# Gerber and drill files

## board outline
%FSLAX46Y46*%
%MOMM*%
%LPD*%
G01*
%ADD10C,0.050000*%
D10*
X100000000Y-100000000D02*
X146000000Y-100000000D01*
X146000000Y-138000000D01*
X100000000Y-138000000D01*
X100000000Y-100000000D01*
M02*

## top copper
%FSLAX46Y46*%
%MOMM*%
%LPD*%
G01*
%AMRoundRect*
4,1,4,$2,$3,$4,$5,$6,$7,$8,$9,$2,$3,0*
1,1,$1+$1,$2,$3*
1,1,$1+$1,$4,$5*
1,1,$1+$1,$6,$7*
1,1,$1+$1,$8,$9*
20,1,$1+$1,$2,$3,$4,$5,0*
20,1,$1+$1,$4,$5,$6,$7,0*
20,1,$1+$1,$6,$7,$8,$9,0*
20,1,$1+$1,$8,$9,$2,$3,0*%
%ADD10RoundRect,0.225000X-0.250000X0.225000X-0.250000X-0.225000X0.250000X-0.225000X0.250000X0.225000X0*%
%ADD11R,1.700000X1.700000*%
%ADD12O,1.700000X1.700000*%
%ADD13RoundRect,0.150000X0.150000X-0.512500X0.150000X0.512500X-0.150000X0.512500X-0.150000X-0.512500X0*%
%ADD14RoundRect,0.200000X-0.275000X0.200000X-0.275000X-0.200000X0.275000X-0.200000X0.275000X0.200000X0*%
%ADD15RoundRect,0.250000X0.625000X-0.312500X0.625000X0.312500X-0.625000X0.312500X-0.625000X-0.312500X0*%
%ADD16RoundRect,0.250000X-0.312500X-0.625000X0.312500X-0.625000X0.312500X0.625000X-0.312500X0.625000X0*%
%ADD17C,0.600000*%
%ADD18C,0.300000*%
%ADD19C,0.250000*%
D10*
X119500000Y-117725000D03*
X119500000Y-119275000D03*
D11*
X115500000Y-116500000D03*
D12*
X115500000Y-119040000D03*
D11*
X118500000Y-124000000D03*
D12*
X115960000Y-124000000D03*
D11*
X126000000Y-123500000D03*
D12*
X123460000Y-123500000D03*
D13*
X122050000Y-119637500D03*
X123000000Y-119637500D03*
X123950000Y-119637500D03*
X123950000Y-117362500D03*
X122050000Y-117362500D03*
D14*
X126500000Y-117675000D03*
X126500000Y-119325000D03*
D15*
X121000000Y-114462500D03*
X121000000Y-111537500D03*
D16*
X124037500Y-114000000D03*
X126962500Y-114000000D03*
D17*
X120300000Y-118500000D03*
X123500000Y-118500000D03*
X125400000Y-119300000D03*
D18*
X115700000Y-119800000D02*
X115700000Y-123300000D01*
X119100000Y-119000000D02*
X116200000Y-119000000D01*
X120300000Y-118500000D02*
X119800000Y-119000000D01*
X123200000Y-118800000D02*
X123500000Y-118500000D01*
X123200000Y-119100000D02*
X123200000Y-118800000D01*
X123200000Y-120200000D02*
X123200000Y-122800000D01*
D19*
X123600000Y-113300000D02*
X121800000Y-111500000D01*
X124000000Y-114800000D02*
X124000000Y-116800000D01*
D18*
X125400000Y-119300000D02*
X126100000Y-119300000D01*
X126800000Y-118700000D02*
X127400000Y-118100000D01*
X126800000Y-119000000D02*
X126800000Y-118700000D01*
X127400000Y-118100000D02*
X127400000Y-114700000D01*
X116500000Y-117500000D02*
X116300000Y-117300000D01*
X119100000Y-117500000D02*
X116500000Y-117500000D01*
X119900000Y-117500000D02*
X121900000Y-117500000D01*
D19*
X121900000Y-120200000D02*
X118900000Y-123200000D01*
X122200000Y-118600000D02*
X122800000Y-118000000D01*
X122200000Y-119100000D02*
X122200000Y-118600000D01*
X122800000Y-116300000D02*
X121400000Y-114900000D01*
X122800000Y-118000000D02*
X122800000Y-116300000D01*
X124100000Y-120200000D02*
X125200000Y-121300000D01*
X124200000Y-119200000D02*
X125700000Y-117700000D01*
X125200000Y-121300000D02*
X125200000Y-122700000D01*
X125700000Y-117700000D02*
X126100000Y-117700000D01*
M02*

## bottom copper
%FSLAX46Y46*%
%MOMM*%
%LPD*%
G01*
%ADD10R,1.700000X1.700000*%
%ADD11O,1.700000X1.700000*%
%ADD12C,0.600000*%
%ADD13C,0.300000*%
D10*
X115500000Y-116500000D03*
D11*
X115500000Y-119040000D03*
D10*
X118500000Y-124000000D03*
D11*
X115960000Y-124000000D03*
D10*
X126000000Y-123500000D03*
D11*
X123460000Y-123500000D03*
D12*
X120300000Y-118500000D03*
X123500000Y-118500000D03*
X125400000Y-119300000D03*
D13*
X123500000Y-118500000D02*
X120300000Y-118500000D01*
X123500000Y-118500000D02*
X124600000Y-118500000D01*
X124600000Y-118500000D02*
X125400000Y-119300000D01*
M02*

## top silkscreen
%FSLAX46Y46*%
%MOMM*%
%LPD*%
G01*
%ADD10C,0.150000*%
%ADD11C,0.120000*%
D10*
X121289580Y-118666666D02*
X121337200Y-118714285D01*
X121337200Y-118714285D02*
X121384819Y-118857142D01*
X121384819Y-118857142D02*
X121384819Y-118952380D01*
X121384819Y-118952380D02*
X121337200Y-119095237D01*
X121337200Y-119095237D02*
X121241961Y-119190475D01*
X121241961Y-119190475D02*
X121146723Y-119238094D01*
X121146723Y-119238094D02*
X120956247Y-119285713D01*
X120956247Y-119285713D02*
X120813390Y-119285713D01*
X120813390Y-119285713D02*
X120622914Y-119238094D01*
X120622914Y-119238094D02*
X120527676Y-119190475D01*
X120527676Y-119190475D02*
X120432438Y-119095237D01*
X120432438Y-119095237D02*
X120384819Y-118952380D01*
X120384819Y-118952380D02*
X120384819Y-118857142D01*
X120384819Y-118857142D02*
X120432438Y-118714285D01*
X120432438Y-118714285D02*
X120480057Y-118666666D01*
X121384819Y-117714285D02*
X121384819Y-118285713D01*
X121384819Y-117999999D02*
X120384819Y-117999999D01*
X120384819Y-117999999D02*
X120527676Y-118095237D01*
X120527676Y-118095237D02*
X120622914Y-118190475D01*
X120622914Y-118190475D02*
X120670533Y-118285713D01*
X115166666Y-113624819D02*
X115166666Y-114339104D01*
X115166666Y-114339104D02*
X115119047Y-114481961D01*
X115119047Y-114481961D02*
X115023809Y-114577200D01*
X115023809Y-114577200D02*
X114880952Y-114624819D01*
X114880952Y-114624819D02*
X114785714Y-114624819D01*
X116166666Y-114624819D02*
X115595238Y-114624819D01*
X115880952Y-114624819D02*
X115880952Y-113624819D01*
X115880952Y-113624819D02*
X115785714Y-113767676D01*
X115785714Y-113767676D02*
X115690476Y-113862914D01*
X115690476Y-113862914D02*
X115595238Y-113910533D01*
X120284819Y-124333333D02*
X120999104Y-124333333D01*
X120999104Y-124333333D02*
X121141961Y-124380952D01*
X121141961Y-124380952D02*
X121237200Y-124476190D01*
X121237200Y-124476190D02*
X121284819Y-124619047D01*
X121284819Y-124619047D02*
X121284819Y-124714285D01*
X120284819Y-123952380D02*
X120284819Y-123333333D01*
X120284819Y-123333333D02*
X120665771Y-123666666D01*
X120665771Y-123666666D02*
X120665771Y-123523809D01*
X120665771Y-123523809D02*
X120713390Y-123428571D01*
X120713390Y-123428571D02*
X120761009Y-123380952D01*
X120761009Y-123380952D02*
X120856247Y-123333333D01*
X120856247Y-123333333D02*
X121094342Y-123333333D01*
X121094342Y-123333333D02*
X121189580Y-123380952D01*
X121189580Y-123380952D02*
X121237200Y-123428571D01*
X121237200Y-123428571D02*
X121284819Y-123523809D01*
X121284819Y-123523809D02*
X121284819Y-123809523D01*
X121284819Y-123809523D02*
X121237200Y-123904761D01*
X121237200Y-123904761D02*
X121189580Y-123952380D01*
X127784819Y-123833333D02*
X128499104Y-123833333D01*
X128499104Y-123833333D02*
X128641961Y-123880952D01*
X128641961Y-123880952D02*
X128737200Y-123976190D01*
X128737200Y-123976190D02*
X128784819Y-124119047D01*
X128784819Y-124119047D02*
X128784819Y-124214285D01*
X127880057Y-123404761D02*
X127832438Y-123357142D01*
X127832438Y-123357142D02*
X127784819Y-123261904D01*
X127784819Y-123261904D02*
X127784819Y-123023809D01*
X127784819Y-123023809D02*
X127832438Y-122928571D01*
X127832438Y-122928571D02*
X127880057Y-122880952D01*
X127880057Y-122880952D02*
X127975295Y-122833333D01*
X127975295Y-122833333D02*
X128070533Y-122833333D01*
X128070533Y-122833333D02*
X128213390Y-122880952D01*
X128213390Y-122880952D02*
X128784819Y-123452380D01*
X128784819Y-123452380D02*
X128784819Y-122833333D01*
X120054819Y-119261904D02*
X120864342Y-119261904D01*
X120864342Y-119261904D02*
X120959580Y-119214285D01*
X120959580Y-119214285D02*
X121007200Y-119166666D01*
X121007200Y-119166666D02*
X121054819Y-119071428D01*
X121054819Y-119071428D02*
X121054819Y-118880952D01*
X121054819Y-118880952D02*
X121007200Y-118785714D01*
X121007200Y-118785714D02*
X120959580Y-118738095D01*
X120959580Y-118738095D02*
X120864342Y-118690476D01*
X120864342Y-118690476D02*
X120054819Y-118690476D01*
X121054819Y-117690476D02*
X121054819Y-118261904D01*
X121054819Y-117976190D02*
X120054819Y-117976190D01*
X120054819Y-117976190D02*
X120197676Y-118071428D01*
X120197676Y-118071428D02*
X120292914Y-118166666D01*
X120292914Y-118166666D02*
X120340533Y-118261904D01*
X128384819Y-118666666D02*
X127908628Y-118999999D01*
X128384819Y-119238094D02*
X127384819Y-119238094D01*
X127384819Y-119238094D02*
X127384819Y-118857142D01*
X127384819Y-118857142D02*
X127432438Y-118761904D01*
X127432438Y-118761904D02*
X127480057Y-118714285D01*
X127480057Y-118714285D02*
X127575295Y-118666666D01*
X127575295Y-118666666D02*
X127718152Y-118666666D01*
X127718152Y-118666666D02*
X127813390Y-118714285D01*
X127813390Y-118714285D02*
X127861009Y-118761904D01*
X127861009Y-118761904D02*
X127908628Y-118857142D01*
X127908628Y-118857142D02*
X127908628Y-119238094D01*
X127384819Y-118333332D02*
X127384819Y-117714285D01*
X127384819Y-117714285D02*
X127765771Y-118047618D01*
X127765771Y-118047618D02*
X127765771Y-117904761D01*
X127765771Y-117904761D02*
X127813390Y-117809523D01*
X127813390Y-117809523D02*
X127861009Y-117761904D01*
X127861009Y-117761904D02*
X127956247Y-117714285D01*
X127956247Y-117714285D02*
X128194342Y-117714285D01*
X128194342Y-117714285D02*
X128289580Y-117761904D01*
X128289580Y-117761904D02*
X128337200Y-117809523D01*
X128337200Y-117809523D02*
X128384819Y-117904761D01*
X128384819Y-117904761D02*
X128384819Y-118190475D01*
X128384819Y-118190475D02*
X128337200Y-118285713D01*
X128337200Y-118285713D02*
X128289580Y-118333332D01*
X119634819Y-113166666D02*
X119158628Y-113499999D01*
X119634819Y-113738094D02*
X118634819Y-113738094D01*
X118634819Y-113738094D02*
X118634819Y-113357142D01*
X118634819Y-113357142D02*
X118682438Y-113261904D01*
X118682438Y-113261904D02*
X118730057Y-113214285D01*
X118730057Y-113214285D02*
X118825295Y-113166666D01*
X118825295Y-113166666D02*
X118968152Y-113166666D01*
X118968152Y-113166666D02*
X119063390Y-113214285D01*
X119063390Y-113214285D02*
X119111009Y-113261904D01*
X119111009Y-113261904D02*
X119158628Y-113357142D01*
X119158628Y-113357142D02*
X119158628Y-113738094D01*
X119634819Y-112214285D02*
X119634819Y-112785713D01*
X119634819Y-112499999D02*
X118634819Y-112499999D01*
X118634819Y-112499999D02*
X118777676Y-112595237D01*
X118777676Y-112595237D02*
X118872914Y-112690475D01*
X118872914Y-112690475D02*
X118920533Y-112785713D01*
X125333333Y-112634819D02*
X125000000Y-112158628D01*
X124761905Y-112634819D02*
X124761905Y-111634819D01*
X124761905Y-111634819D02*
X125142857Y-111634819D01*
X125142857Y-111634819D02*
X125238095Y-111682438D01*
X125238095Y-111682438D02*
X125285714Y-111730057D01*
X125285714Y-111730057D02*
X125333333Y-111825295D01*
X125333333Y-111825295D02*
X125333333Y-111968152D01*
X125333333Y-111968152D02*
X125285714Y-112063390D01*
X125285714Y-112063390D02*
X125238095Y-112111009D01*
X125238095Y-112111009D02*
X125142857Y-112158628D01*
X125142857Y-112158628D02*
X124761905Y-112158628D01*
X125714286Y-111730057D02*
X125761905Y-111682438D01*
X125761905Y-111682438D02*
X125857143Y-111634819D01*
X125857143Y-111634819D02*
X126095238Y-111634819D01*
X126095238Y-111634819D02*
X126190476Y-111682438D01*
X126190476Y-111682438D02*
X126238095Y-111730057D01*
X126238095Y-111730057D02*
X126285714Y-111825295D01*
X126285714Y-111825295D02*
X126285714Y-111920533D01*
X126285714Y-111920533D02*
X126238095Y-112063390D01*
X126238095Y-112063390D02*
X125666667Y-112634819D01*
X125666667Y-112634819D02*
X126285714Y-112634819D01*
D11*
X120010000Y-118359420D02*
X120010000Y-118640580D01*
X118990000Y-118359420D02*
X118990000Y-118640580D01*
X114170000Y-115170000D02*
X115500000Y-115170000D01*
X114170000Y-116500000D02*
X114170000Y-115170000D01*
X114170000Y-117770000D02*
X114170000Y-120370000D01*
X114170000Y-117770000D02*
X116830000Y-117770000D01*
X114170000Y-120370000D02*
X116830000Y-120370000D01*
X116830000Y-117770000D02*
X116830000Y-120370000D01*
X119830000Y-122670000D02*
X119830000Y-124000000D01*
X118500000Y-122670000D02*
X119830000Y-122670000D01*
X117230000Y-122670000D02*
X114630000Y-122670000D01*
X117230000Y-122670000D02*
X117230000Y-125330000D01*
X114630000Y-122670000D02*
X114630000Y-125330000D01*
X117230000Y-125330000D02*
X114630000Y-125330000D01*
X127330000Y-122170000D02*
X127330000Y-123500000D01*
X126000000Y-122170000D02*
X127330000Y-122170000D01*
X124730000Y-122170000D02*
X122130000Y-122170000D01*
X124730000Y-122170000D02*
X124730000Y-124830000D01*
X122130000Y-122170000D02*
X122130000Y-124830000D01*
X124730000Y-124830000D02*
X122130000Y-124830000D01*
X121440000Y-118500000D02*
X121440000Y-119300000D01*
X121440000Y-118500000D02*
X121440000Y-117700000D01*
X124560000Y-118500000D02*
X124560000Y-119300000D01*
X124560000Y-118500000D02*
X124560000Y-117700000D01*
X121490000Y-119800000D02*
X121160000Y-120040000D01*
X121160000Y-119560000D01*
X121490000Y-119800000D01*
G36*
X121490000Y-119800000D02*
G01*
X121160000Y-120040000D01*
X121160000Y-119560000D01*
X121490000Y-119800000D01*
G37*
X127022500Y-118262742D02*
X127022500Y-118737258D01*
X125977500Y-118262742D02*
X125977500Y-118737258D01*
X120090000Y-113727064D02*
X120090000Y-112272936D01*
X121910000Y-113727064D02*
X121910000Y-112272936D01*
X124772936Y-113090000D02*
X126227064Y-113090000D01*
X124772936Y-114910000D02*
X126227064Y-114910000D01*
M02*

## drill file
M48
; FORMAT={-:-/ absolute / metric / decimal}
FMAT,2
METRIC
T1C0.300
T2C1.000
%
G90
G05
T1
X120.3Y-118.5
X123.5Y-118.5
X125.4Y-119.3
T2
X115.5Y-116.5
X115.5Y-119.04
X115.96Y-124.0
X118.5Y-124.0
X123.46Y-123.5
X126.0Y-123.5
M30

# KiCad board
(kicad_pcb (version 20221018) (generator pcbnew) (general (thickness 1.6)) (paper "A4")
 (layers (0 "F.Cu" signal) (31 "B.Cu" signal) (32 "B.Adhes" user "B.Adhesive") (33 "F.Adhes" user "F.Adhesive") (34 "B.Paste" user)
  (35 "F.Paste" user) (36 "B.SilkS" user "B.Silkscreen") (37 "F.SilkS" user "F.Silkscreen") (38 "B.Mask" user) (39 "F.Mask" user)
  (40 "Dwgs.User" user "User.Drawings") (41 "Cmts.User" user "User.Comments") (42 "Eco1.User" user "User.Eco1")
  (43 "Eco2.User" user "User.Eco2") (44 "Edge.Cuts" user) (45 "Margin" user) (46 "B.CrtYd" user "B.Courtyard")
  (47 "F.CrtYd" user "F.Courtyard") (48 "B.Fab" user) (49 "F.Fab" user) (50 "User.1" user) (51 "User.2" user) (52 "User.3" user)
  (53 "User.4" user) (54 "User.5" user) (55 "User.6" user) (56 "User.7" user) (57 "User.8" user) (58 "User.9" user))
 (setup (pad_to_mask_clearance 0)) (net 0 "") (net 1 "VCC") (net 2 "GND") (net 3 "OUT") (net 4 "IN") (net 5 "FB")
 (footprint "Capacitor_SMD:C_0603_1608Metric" (layer "F.Cu") (at 119.5 118.5 -90)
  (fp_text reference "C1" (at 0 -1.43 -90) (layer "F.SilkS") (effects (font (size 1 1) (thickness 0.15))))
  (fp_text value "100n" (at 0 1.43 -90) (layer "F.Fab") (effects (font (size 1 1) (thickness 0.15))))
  (fp_line (start -0.14058 -0.51) (end 0.14058 -0.51) (stroke (width 0.12) (type solid)) (layer "F.SilkS"))
  (fp_line (start -0.14058 0.51) (end 0.14058 0.51) (stroke (width 0.12) (type solid)) (layer "F.SilkS"))
  (pad "1" smd roundrect (at -0.775 0 270) (size 0.9 0.95) (layers "F.Cu" "F.Paste" "F.Mask") (roundrect_rratio 0.25) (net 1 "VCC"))
  (pad "2" smd roundrect (at 0.775 0 270) (size 0.9 0.95) (layers "F.Cu" "F.Paste" "F.Mask") (roundrect_rratio 0.25) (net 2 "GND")))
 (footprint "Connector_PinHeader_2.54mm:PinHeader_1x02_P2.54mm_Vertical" (layer "F.Cu") (at 115.5 116.5)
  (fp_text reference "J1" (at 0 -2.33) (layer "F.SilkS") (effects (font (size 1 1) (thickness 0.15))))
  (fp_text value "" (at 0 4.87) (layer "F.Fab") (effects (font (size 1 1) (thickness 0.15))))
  (fp_line (start -1.33 -1.33) (end 0 -1.33) (stroke (width 0.12) (type solid)) (layer "F.SilkS"))
  (fp_line (start -1.33 0) (end -1.33 -1.33) (stroke (width 0.12) (type solid)) (layer "F.SilkS"))
  (fp_line (start -1.33 1.27) (end -1.33 3.87) (stroke (width 0.12) (type solid)) (layer "F.SilkS"))
  (fp_line (start -1.33 1.27) (end 1.33 1.27) (stroke (width 0.12) (type solid)) (layer "F.SilkS"))
  (fp_line (start -1.33 3.87) (end 1.33 3.87) (stroke (width 0.12) (type solid)) (layer "F.SilkS"))
  (fp_line (start 1.33 1.27) (end 1.33 3.87) (stroke (width 0.12) (type solid)) (layer "F.SilkS"))
  (pad "1" thru_hole rect (at 0 0) (size 1.7 1.7) (drill 1) (layers "*.Cu" "*.Mask") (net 1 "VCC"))
  (pad "2" thru_hole oval (at 0 2.54) (size 1.7 1.7) (drill 1) (layers "*.Cu" "*.Mask") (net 2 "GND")))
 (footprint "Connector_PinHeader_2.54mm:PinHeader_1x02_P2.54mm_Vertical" (layer "F.Cu") (at 118.5 124 -90)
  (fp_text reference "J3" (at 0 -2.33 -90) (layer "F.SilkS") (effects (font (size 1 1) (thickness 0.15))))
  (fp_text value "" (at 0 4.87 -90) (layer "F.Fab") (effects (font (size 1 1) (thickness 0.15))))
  (fp_line (start -1.33 -1.33) (end 0 -1.33) (stroke (width 0.12) (type solid)) (layer "F.SilkS"))
  (fp_line (start -1.33 0) (end -1.33 -1.33) (stroke (width 0.12) (type solid)) (layer "F.SilkS"))
  (fp_line (start -1.33 1.27) (end -1.33 3.87) (stroke (width 0.12) (type solid)) (layer "F.SilkS"))
  (fp_line (start -1.33 1.27) (end 1.33 1.27) (stroke (width 0.12) (type solid)) (layer "F.SilkS"))
  (fp_line (start -1.33 3.87) (end 1.33 3.87) (stroke (width 0.12) (type solid)) (layer "F.SilkS"))
  (fp_line (start 1.33 1.27) (end 1.33 3.87) (stroke (width 0.12) (type solid)) (layer "F.SilkS"))
  (pad "1" thru_hole rect (at 0 0 270) (size 1.7 1.7) (drill 1) (layers "*.Cu" "*.Mask") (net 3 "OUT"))
  (pad "2" thru_hole oval (at 0 2.54 270) (size 1.7 1.7) (drill 1) (layers "*.Cu" "*.Mask") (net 2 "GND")))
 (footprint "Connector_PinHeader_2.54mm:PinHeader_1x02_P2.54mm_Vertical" (layer "F.Cu") (at 126 123.5 -90)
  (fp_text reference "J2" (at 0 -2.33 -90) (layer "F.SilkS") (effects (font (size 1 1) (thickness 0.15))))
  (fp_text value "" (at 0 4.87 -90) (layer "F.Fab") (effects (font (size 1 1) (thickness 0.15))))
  (fp_line (start -1.33 -1.33) (end 0 -1.33) (stroke (width 0.12) (type solid)) (layer "F.SilkS"))
  (fp_line (start -1.33 0) (end -1.33 -1.33) (stroke (width 0.12) (type solid)) (layer "F.SilkS"))
  (fp_line (start -1.33 1.27) (end -1.33 3.87) (stroke (width 0.12) (type solid)) (layer "F.SilkS"))
  (fp_line (start -1.33 1.27) (end 1.33 1.27) (stroke (width 0.12) (type solid)) (layer "F.SilkS"))
  (fp_line (start -1.33 3.87) (end 1.33 3.87) (stroke (width 0.12) (type solid)) (layer "F.SilkS"))
  (fp_line (start 1.33 1.27) (end 1.33 3.87) (stroke (width 0.12) (type solid)) (layer "F.SilkS"))
  (pad "1" thru_hole rect (at 0 0 270) (size 1.7 1.7) (drill 1) (layers "*.Cu" "*.Mask") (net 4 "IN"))
  (pad "2" thru_hole oval (at 0 2.54 270) (size 1.7 1.7) (drill 1) (layers "*.Cu" "*.Mask") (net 2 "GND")))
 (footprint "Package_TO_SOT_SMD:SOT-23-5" (layer "F.Cu") (at 123 118.5 90)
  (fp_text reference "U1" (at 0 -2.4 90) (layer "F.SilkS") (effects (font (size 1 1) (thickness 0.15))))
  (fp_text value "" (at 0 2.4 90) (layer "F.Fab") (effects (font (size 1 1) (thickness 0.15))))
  (fp_line (start 0 -1.56) (end -0.8 -1.56) (stroke (width 0.12) (type solid)) (layer "F.SilkS"))
  (fp_line (start 0 -1.56) (end 0.8 -1.56) (stroke (width 0.12) (type solid)) (layer "F.SilkS"))
  (fp_line (start 0 1.56) (end -0.8 1.56) (stroke (width 0.12) (type solid)) (layer "F.SilkS"))
  (fp_line (start 0 1.56) (end 0.8 1.56) (stroke (width 0.12) (type solid)) (layer "F.SilkS"))
  (fp_poly
   (pts (xy -1.3 -1.51) (xy -1.54 -1.84) (xy -1.06 -1.84) (xy -1.3 -1.51)) (stroke (width 0.12) (type solid)) (fill solid) (layer "F.SilkS"))
  (pad "1" smd roundrect (at -1.1375 -0.95 90) (size 1.325 0.6) (layers "F.Cu" "F.Paste" "F.Mask") (roundrect_rratio 0.25) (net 3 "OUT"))
  (pad "2" smd roundrect (at -1.1375 0 90) (size 1.325 0.6) (layers "F.Cu" "F.Paste" "F.Mask") (roundrect_rratio 0.25) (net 2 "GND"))
  (pad "3" smd roundrect (at -1.1375 0.95 90) (size 1.325 0.6) (layers "F.Cu" "F.Paste" "F.Mask") (roundrect_rratio 0.25) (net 4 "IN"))
  (pad "4" smd roundrect (at 1.1375 0.95 90) (size 1.325 0.6) (layers "F.Cu" "F.Paste" "F.Mask") (roundrect_rratio 0.25) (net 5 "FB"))
  (pad "5" smd roundrect (at 1.1375 -0.95 90) (size 1.325 0.6) (layers "F.Cu" "F.Paste" "F.Mask") (roundrect_rratio 0.25) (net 1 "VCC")))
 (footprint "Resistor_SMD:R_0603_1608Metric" (layer "F.Cu") (at 126.5 118.5 -90)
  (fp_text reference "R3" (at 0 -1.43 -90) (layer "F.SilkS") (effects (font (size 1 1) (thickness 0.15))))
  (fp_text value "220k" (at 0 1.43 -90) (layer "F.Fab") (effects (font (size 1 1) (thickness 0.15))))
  (fp_line (start -0.237258 -0.5225) (end 0.237258 -0.5225) (stroke (width 0.12) (type solid)) (layer "F.SilkS"))
  (fp_line (start -0.237258 0.5225) (end 0.237258 0.5225) (stroke (width 0.12) (type solid)) (layer "F.SilkS"))
  (pad "1" smd roundrect (at -0.825 0 270) (size 0.8 0.95) (layers "F.Cu" "F.Paste" "F.Mask") (roundrect_rratio 0.25) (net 4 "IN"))
  (pad "2" smd roundrect (at 0.825 0 270) (size 0.8 0.95) (layers "F.Cu" "F.Paste" "F.Mask") (roundrect_rratio 0.25) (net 2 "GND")))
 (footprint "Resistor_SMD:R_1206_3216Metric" (layer "F.Cu") (at 121 113 90)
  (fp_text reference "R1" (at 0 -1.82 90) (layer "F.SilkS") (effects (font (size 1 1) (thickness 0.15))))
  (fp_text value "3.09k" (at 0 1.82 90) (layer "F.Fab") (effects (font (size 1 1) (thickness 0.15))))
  (fp_line (start -0.727064 -0.91) (end 0.727064 -0.91) (stroke (width 0.12) (type solid)) (layer "F.SilkS"))
  (fp_line (start -0.727064 0.91) (end 0.727064 0.91) (stroke (width 0.12) (type solid)) (layer "F.SilkS"))
  (pad "1" smd roundrect (at -1.4625 0 90) (size 1.125 1.75) (layers "F.Cu" "F.Paste" "F.Mask") (roundrect_rratio 0.222222) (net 3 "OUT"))
  (pad "2" smd roundrect (at 1.4625 0 90) (size 1.125 1.75) (layers "F.Cu" "F.Paste" "F.Mask") (roundrect_rratio 0.222222) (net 5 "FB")))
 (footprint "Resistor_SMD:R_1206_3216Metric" (layer "F.Cu") (at 125.5 114)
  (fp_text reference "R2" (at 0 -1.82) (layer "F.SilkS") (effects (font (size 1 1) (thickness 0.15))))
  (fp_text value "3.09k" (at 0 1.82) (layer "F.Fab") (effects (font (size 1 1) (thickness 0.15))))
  (fp_line (start -0.727064 -0.91) (end 0.727064 -0.91) (stroke (width 0.12) (type solid)) (layer "F.SilkS"))
  (fp_line (start -0.727064 0.91) (end 0.727064 0.91) (stroke (width 0.12) (type solid)) (layer "F.SilkS"))
  (pad "1" smd roundrect (at -1.4625 0) (size 1.125 1.75) (layers "F.Cu" "F.Paste" "F.Mask") (roundrect_rratio 0.222222) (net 5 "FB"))
  (pad "2" smd roundrect (at 1.4625 0) (size 1.125 1.75) (layers "F.Cu" "F.Paste" "F.Mask") (roundrect_rratio 0.222222) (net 2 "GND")))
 (gr_rect (start 100 100) (end 146 138) (stroke (width 0.05) (type default)) (fill none) (layer "Edge.Cuts"))
 (segment (start 115.7 119.8) (end 115.7 123.3) (width 0.3) (layer "F.Cu") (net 2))
 (segment (start 119.1 119) (end 116.2 119) (width 0.3) (layer "F.Cu") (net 2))
 (segment (start 120.3 118.5) (end 119.8 119) (width 0.3) (layer "F.Cu") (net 2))
 (segment (start 123.2 118.8) (end 123.5 118.5) (width 0.3) (layer "F.Cu") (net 2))
 (segment (start 123.2 119.1) (end 123.2 118.8) (width 0.3) (layer "F.Cu") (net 2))
 (segment (start 123.2 120.2) (end 123.2 122.8) (width 0.3) (layer "F.Cu") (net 2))
 (segment (start 123.6 113.3) (end 121.8 111.5) (width 0.25) (layer "F.Cu") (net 5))
 (segment (start 124 114.8) (end 124 116.8) (width 0.25) (layer "F.Cu") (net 5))
 (segment (start 125.4 119.3) (end 126.1 119.3) (width 0.3) (layer "F.Cu") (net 2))
 (segment (start 126.8 118.7) (end 127.4 118.1) (width 0.3) (layer "F.Cu") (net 2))
 (segment (start 126.8 119) (end 126.8 118.7) (width 0.3) (layer "F.Cu") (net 2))
 (segment (start 127.4 118.1) (end 127.4 114.7) (width 0.3) (layer "F.Cu") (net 2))
 (via (at 120.3 118.5) (size 0.6) (drill 0.3) (layers "F.Cu" "B.Cu") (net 2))
 (via (at 123.5 118.5) (size 0.6) (drill 0.3) (layers "F.Cu" "B.Cu") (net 2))
 (via (at 125.4 119.3) (size 0.6) (drill 0.3) (layers "F.Cu" "B.Cu") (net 2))
 (segment (start 116.5 117.5) (end 116.3 117.3) (width 0.3) (layer "F.Cu") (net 1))
 (segment (start 119.1 117.5) (end 116.5 117.5) (width 0.3) (layer "F.Cu") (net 1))
 (segment (start 119.9 117.5) (end 121.9 117.5) (width 0.3) (layer "F.Cu") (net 1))
 (segment (start 121.9 120.2) (end 118.9 123.2) (width 0.25) (layer "F.Cu") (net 3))
 (segment (start 122.2 118.6) (end 122.8 118) (width 0.25) (layer "F.Cu") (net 3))
 (segment (start 122.2 119.1) (end 122.2 118.6) (width 0.25) (layer "F.Cu") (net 3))
 (segment (start 122.8 116.3) (end 121.4 114.9) (width 0.25) (layer "F.Cu") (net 3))
 (segment (start 122.8 118) (end 122.8 116.3) (width 0.25) (layer "F.Cu") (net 3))
 (segment (start 123.5 118.5) (end 120.3 118.5) (width 0.3) (layer "B.Cu") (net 2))
 (segment (start 123.5 118.5) (end 124.6 118.5) (width 0.3) (layer "B.Cu") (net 2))
 (segment (start 124.1 120.2) (end 125.2 121.3) (width 0.25) (layer "F.Cu") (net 4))
 (segment (start 124.2 119.2) (end 125.7 117.7) (width 0.25) (layer "F.Cu") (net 4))
 (segment (start 124.6 118.5) (end 125.4 119.3) (width 0.3) (layer "B.Cu") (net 2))
 (segment (start 125.2 121.3) (end 125.2 122.7) (width 0.25) (layer "F.Cu") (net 4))
 (segment (start 125.7 117.7) (end 126.1 117.7) (width 0.25) (layer "F.Cu") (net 4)))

